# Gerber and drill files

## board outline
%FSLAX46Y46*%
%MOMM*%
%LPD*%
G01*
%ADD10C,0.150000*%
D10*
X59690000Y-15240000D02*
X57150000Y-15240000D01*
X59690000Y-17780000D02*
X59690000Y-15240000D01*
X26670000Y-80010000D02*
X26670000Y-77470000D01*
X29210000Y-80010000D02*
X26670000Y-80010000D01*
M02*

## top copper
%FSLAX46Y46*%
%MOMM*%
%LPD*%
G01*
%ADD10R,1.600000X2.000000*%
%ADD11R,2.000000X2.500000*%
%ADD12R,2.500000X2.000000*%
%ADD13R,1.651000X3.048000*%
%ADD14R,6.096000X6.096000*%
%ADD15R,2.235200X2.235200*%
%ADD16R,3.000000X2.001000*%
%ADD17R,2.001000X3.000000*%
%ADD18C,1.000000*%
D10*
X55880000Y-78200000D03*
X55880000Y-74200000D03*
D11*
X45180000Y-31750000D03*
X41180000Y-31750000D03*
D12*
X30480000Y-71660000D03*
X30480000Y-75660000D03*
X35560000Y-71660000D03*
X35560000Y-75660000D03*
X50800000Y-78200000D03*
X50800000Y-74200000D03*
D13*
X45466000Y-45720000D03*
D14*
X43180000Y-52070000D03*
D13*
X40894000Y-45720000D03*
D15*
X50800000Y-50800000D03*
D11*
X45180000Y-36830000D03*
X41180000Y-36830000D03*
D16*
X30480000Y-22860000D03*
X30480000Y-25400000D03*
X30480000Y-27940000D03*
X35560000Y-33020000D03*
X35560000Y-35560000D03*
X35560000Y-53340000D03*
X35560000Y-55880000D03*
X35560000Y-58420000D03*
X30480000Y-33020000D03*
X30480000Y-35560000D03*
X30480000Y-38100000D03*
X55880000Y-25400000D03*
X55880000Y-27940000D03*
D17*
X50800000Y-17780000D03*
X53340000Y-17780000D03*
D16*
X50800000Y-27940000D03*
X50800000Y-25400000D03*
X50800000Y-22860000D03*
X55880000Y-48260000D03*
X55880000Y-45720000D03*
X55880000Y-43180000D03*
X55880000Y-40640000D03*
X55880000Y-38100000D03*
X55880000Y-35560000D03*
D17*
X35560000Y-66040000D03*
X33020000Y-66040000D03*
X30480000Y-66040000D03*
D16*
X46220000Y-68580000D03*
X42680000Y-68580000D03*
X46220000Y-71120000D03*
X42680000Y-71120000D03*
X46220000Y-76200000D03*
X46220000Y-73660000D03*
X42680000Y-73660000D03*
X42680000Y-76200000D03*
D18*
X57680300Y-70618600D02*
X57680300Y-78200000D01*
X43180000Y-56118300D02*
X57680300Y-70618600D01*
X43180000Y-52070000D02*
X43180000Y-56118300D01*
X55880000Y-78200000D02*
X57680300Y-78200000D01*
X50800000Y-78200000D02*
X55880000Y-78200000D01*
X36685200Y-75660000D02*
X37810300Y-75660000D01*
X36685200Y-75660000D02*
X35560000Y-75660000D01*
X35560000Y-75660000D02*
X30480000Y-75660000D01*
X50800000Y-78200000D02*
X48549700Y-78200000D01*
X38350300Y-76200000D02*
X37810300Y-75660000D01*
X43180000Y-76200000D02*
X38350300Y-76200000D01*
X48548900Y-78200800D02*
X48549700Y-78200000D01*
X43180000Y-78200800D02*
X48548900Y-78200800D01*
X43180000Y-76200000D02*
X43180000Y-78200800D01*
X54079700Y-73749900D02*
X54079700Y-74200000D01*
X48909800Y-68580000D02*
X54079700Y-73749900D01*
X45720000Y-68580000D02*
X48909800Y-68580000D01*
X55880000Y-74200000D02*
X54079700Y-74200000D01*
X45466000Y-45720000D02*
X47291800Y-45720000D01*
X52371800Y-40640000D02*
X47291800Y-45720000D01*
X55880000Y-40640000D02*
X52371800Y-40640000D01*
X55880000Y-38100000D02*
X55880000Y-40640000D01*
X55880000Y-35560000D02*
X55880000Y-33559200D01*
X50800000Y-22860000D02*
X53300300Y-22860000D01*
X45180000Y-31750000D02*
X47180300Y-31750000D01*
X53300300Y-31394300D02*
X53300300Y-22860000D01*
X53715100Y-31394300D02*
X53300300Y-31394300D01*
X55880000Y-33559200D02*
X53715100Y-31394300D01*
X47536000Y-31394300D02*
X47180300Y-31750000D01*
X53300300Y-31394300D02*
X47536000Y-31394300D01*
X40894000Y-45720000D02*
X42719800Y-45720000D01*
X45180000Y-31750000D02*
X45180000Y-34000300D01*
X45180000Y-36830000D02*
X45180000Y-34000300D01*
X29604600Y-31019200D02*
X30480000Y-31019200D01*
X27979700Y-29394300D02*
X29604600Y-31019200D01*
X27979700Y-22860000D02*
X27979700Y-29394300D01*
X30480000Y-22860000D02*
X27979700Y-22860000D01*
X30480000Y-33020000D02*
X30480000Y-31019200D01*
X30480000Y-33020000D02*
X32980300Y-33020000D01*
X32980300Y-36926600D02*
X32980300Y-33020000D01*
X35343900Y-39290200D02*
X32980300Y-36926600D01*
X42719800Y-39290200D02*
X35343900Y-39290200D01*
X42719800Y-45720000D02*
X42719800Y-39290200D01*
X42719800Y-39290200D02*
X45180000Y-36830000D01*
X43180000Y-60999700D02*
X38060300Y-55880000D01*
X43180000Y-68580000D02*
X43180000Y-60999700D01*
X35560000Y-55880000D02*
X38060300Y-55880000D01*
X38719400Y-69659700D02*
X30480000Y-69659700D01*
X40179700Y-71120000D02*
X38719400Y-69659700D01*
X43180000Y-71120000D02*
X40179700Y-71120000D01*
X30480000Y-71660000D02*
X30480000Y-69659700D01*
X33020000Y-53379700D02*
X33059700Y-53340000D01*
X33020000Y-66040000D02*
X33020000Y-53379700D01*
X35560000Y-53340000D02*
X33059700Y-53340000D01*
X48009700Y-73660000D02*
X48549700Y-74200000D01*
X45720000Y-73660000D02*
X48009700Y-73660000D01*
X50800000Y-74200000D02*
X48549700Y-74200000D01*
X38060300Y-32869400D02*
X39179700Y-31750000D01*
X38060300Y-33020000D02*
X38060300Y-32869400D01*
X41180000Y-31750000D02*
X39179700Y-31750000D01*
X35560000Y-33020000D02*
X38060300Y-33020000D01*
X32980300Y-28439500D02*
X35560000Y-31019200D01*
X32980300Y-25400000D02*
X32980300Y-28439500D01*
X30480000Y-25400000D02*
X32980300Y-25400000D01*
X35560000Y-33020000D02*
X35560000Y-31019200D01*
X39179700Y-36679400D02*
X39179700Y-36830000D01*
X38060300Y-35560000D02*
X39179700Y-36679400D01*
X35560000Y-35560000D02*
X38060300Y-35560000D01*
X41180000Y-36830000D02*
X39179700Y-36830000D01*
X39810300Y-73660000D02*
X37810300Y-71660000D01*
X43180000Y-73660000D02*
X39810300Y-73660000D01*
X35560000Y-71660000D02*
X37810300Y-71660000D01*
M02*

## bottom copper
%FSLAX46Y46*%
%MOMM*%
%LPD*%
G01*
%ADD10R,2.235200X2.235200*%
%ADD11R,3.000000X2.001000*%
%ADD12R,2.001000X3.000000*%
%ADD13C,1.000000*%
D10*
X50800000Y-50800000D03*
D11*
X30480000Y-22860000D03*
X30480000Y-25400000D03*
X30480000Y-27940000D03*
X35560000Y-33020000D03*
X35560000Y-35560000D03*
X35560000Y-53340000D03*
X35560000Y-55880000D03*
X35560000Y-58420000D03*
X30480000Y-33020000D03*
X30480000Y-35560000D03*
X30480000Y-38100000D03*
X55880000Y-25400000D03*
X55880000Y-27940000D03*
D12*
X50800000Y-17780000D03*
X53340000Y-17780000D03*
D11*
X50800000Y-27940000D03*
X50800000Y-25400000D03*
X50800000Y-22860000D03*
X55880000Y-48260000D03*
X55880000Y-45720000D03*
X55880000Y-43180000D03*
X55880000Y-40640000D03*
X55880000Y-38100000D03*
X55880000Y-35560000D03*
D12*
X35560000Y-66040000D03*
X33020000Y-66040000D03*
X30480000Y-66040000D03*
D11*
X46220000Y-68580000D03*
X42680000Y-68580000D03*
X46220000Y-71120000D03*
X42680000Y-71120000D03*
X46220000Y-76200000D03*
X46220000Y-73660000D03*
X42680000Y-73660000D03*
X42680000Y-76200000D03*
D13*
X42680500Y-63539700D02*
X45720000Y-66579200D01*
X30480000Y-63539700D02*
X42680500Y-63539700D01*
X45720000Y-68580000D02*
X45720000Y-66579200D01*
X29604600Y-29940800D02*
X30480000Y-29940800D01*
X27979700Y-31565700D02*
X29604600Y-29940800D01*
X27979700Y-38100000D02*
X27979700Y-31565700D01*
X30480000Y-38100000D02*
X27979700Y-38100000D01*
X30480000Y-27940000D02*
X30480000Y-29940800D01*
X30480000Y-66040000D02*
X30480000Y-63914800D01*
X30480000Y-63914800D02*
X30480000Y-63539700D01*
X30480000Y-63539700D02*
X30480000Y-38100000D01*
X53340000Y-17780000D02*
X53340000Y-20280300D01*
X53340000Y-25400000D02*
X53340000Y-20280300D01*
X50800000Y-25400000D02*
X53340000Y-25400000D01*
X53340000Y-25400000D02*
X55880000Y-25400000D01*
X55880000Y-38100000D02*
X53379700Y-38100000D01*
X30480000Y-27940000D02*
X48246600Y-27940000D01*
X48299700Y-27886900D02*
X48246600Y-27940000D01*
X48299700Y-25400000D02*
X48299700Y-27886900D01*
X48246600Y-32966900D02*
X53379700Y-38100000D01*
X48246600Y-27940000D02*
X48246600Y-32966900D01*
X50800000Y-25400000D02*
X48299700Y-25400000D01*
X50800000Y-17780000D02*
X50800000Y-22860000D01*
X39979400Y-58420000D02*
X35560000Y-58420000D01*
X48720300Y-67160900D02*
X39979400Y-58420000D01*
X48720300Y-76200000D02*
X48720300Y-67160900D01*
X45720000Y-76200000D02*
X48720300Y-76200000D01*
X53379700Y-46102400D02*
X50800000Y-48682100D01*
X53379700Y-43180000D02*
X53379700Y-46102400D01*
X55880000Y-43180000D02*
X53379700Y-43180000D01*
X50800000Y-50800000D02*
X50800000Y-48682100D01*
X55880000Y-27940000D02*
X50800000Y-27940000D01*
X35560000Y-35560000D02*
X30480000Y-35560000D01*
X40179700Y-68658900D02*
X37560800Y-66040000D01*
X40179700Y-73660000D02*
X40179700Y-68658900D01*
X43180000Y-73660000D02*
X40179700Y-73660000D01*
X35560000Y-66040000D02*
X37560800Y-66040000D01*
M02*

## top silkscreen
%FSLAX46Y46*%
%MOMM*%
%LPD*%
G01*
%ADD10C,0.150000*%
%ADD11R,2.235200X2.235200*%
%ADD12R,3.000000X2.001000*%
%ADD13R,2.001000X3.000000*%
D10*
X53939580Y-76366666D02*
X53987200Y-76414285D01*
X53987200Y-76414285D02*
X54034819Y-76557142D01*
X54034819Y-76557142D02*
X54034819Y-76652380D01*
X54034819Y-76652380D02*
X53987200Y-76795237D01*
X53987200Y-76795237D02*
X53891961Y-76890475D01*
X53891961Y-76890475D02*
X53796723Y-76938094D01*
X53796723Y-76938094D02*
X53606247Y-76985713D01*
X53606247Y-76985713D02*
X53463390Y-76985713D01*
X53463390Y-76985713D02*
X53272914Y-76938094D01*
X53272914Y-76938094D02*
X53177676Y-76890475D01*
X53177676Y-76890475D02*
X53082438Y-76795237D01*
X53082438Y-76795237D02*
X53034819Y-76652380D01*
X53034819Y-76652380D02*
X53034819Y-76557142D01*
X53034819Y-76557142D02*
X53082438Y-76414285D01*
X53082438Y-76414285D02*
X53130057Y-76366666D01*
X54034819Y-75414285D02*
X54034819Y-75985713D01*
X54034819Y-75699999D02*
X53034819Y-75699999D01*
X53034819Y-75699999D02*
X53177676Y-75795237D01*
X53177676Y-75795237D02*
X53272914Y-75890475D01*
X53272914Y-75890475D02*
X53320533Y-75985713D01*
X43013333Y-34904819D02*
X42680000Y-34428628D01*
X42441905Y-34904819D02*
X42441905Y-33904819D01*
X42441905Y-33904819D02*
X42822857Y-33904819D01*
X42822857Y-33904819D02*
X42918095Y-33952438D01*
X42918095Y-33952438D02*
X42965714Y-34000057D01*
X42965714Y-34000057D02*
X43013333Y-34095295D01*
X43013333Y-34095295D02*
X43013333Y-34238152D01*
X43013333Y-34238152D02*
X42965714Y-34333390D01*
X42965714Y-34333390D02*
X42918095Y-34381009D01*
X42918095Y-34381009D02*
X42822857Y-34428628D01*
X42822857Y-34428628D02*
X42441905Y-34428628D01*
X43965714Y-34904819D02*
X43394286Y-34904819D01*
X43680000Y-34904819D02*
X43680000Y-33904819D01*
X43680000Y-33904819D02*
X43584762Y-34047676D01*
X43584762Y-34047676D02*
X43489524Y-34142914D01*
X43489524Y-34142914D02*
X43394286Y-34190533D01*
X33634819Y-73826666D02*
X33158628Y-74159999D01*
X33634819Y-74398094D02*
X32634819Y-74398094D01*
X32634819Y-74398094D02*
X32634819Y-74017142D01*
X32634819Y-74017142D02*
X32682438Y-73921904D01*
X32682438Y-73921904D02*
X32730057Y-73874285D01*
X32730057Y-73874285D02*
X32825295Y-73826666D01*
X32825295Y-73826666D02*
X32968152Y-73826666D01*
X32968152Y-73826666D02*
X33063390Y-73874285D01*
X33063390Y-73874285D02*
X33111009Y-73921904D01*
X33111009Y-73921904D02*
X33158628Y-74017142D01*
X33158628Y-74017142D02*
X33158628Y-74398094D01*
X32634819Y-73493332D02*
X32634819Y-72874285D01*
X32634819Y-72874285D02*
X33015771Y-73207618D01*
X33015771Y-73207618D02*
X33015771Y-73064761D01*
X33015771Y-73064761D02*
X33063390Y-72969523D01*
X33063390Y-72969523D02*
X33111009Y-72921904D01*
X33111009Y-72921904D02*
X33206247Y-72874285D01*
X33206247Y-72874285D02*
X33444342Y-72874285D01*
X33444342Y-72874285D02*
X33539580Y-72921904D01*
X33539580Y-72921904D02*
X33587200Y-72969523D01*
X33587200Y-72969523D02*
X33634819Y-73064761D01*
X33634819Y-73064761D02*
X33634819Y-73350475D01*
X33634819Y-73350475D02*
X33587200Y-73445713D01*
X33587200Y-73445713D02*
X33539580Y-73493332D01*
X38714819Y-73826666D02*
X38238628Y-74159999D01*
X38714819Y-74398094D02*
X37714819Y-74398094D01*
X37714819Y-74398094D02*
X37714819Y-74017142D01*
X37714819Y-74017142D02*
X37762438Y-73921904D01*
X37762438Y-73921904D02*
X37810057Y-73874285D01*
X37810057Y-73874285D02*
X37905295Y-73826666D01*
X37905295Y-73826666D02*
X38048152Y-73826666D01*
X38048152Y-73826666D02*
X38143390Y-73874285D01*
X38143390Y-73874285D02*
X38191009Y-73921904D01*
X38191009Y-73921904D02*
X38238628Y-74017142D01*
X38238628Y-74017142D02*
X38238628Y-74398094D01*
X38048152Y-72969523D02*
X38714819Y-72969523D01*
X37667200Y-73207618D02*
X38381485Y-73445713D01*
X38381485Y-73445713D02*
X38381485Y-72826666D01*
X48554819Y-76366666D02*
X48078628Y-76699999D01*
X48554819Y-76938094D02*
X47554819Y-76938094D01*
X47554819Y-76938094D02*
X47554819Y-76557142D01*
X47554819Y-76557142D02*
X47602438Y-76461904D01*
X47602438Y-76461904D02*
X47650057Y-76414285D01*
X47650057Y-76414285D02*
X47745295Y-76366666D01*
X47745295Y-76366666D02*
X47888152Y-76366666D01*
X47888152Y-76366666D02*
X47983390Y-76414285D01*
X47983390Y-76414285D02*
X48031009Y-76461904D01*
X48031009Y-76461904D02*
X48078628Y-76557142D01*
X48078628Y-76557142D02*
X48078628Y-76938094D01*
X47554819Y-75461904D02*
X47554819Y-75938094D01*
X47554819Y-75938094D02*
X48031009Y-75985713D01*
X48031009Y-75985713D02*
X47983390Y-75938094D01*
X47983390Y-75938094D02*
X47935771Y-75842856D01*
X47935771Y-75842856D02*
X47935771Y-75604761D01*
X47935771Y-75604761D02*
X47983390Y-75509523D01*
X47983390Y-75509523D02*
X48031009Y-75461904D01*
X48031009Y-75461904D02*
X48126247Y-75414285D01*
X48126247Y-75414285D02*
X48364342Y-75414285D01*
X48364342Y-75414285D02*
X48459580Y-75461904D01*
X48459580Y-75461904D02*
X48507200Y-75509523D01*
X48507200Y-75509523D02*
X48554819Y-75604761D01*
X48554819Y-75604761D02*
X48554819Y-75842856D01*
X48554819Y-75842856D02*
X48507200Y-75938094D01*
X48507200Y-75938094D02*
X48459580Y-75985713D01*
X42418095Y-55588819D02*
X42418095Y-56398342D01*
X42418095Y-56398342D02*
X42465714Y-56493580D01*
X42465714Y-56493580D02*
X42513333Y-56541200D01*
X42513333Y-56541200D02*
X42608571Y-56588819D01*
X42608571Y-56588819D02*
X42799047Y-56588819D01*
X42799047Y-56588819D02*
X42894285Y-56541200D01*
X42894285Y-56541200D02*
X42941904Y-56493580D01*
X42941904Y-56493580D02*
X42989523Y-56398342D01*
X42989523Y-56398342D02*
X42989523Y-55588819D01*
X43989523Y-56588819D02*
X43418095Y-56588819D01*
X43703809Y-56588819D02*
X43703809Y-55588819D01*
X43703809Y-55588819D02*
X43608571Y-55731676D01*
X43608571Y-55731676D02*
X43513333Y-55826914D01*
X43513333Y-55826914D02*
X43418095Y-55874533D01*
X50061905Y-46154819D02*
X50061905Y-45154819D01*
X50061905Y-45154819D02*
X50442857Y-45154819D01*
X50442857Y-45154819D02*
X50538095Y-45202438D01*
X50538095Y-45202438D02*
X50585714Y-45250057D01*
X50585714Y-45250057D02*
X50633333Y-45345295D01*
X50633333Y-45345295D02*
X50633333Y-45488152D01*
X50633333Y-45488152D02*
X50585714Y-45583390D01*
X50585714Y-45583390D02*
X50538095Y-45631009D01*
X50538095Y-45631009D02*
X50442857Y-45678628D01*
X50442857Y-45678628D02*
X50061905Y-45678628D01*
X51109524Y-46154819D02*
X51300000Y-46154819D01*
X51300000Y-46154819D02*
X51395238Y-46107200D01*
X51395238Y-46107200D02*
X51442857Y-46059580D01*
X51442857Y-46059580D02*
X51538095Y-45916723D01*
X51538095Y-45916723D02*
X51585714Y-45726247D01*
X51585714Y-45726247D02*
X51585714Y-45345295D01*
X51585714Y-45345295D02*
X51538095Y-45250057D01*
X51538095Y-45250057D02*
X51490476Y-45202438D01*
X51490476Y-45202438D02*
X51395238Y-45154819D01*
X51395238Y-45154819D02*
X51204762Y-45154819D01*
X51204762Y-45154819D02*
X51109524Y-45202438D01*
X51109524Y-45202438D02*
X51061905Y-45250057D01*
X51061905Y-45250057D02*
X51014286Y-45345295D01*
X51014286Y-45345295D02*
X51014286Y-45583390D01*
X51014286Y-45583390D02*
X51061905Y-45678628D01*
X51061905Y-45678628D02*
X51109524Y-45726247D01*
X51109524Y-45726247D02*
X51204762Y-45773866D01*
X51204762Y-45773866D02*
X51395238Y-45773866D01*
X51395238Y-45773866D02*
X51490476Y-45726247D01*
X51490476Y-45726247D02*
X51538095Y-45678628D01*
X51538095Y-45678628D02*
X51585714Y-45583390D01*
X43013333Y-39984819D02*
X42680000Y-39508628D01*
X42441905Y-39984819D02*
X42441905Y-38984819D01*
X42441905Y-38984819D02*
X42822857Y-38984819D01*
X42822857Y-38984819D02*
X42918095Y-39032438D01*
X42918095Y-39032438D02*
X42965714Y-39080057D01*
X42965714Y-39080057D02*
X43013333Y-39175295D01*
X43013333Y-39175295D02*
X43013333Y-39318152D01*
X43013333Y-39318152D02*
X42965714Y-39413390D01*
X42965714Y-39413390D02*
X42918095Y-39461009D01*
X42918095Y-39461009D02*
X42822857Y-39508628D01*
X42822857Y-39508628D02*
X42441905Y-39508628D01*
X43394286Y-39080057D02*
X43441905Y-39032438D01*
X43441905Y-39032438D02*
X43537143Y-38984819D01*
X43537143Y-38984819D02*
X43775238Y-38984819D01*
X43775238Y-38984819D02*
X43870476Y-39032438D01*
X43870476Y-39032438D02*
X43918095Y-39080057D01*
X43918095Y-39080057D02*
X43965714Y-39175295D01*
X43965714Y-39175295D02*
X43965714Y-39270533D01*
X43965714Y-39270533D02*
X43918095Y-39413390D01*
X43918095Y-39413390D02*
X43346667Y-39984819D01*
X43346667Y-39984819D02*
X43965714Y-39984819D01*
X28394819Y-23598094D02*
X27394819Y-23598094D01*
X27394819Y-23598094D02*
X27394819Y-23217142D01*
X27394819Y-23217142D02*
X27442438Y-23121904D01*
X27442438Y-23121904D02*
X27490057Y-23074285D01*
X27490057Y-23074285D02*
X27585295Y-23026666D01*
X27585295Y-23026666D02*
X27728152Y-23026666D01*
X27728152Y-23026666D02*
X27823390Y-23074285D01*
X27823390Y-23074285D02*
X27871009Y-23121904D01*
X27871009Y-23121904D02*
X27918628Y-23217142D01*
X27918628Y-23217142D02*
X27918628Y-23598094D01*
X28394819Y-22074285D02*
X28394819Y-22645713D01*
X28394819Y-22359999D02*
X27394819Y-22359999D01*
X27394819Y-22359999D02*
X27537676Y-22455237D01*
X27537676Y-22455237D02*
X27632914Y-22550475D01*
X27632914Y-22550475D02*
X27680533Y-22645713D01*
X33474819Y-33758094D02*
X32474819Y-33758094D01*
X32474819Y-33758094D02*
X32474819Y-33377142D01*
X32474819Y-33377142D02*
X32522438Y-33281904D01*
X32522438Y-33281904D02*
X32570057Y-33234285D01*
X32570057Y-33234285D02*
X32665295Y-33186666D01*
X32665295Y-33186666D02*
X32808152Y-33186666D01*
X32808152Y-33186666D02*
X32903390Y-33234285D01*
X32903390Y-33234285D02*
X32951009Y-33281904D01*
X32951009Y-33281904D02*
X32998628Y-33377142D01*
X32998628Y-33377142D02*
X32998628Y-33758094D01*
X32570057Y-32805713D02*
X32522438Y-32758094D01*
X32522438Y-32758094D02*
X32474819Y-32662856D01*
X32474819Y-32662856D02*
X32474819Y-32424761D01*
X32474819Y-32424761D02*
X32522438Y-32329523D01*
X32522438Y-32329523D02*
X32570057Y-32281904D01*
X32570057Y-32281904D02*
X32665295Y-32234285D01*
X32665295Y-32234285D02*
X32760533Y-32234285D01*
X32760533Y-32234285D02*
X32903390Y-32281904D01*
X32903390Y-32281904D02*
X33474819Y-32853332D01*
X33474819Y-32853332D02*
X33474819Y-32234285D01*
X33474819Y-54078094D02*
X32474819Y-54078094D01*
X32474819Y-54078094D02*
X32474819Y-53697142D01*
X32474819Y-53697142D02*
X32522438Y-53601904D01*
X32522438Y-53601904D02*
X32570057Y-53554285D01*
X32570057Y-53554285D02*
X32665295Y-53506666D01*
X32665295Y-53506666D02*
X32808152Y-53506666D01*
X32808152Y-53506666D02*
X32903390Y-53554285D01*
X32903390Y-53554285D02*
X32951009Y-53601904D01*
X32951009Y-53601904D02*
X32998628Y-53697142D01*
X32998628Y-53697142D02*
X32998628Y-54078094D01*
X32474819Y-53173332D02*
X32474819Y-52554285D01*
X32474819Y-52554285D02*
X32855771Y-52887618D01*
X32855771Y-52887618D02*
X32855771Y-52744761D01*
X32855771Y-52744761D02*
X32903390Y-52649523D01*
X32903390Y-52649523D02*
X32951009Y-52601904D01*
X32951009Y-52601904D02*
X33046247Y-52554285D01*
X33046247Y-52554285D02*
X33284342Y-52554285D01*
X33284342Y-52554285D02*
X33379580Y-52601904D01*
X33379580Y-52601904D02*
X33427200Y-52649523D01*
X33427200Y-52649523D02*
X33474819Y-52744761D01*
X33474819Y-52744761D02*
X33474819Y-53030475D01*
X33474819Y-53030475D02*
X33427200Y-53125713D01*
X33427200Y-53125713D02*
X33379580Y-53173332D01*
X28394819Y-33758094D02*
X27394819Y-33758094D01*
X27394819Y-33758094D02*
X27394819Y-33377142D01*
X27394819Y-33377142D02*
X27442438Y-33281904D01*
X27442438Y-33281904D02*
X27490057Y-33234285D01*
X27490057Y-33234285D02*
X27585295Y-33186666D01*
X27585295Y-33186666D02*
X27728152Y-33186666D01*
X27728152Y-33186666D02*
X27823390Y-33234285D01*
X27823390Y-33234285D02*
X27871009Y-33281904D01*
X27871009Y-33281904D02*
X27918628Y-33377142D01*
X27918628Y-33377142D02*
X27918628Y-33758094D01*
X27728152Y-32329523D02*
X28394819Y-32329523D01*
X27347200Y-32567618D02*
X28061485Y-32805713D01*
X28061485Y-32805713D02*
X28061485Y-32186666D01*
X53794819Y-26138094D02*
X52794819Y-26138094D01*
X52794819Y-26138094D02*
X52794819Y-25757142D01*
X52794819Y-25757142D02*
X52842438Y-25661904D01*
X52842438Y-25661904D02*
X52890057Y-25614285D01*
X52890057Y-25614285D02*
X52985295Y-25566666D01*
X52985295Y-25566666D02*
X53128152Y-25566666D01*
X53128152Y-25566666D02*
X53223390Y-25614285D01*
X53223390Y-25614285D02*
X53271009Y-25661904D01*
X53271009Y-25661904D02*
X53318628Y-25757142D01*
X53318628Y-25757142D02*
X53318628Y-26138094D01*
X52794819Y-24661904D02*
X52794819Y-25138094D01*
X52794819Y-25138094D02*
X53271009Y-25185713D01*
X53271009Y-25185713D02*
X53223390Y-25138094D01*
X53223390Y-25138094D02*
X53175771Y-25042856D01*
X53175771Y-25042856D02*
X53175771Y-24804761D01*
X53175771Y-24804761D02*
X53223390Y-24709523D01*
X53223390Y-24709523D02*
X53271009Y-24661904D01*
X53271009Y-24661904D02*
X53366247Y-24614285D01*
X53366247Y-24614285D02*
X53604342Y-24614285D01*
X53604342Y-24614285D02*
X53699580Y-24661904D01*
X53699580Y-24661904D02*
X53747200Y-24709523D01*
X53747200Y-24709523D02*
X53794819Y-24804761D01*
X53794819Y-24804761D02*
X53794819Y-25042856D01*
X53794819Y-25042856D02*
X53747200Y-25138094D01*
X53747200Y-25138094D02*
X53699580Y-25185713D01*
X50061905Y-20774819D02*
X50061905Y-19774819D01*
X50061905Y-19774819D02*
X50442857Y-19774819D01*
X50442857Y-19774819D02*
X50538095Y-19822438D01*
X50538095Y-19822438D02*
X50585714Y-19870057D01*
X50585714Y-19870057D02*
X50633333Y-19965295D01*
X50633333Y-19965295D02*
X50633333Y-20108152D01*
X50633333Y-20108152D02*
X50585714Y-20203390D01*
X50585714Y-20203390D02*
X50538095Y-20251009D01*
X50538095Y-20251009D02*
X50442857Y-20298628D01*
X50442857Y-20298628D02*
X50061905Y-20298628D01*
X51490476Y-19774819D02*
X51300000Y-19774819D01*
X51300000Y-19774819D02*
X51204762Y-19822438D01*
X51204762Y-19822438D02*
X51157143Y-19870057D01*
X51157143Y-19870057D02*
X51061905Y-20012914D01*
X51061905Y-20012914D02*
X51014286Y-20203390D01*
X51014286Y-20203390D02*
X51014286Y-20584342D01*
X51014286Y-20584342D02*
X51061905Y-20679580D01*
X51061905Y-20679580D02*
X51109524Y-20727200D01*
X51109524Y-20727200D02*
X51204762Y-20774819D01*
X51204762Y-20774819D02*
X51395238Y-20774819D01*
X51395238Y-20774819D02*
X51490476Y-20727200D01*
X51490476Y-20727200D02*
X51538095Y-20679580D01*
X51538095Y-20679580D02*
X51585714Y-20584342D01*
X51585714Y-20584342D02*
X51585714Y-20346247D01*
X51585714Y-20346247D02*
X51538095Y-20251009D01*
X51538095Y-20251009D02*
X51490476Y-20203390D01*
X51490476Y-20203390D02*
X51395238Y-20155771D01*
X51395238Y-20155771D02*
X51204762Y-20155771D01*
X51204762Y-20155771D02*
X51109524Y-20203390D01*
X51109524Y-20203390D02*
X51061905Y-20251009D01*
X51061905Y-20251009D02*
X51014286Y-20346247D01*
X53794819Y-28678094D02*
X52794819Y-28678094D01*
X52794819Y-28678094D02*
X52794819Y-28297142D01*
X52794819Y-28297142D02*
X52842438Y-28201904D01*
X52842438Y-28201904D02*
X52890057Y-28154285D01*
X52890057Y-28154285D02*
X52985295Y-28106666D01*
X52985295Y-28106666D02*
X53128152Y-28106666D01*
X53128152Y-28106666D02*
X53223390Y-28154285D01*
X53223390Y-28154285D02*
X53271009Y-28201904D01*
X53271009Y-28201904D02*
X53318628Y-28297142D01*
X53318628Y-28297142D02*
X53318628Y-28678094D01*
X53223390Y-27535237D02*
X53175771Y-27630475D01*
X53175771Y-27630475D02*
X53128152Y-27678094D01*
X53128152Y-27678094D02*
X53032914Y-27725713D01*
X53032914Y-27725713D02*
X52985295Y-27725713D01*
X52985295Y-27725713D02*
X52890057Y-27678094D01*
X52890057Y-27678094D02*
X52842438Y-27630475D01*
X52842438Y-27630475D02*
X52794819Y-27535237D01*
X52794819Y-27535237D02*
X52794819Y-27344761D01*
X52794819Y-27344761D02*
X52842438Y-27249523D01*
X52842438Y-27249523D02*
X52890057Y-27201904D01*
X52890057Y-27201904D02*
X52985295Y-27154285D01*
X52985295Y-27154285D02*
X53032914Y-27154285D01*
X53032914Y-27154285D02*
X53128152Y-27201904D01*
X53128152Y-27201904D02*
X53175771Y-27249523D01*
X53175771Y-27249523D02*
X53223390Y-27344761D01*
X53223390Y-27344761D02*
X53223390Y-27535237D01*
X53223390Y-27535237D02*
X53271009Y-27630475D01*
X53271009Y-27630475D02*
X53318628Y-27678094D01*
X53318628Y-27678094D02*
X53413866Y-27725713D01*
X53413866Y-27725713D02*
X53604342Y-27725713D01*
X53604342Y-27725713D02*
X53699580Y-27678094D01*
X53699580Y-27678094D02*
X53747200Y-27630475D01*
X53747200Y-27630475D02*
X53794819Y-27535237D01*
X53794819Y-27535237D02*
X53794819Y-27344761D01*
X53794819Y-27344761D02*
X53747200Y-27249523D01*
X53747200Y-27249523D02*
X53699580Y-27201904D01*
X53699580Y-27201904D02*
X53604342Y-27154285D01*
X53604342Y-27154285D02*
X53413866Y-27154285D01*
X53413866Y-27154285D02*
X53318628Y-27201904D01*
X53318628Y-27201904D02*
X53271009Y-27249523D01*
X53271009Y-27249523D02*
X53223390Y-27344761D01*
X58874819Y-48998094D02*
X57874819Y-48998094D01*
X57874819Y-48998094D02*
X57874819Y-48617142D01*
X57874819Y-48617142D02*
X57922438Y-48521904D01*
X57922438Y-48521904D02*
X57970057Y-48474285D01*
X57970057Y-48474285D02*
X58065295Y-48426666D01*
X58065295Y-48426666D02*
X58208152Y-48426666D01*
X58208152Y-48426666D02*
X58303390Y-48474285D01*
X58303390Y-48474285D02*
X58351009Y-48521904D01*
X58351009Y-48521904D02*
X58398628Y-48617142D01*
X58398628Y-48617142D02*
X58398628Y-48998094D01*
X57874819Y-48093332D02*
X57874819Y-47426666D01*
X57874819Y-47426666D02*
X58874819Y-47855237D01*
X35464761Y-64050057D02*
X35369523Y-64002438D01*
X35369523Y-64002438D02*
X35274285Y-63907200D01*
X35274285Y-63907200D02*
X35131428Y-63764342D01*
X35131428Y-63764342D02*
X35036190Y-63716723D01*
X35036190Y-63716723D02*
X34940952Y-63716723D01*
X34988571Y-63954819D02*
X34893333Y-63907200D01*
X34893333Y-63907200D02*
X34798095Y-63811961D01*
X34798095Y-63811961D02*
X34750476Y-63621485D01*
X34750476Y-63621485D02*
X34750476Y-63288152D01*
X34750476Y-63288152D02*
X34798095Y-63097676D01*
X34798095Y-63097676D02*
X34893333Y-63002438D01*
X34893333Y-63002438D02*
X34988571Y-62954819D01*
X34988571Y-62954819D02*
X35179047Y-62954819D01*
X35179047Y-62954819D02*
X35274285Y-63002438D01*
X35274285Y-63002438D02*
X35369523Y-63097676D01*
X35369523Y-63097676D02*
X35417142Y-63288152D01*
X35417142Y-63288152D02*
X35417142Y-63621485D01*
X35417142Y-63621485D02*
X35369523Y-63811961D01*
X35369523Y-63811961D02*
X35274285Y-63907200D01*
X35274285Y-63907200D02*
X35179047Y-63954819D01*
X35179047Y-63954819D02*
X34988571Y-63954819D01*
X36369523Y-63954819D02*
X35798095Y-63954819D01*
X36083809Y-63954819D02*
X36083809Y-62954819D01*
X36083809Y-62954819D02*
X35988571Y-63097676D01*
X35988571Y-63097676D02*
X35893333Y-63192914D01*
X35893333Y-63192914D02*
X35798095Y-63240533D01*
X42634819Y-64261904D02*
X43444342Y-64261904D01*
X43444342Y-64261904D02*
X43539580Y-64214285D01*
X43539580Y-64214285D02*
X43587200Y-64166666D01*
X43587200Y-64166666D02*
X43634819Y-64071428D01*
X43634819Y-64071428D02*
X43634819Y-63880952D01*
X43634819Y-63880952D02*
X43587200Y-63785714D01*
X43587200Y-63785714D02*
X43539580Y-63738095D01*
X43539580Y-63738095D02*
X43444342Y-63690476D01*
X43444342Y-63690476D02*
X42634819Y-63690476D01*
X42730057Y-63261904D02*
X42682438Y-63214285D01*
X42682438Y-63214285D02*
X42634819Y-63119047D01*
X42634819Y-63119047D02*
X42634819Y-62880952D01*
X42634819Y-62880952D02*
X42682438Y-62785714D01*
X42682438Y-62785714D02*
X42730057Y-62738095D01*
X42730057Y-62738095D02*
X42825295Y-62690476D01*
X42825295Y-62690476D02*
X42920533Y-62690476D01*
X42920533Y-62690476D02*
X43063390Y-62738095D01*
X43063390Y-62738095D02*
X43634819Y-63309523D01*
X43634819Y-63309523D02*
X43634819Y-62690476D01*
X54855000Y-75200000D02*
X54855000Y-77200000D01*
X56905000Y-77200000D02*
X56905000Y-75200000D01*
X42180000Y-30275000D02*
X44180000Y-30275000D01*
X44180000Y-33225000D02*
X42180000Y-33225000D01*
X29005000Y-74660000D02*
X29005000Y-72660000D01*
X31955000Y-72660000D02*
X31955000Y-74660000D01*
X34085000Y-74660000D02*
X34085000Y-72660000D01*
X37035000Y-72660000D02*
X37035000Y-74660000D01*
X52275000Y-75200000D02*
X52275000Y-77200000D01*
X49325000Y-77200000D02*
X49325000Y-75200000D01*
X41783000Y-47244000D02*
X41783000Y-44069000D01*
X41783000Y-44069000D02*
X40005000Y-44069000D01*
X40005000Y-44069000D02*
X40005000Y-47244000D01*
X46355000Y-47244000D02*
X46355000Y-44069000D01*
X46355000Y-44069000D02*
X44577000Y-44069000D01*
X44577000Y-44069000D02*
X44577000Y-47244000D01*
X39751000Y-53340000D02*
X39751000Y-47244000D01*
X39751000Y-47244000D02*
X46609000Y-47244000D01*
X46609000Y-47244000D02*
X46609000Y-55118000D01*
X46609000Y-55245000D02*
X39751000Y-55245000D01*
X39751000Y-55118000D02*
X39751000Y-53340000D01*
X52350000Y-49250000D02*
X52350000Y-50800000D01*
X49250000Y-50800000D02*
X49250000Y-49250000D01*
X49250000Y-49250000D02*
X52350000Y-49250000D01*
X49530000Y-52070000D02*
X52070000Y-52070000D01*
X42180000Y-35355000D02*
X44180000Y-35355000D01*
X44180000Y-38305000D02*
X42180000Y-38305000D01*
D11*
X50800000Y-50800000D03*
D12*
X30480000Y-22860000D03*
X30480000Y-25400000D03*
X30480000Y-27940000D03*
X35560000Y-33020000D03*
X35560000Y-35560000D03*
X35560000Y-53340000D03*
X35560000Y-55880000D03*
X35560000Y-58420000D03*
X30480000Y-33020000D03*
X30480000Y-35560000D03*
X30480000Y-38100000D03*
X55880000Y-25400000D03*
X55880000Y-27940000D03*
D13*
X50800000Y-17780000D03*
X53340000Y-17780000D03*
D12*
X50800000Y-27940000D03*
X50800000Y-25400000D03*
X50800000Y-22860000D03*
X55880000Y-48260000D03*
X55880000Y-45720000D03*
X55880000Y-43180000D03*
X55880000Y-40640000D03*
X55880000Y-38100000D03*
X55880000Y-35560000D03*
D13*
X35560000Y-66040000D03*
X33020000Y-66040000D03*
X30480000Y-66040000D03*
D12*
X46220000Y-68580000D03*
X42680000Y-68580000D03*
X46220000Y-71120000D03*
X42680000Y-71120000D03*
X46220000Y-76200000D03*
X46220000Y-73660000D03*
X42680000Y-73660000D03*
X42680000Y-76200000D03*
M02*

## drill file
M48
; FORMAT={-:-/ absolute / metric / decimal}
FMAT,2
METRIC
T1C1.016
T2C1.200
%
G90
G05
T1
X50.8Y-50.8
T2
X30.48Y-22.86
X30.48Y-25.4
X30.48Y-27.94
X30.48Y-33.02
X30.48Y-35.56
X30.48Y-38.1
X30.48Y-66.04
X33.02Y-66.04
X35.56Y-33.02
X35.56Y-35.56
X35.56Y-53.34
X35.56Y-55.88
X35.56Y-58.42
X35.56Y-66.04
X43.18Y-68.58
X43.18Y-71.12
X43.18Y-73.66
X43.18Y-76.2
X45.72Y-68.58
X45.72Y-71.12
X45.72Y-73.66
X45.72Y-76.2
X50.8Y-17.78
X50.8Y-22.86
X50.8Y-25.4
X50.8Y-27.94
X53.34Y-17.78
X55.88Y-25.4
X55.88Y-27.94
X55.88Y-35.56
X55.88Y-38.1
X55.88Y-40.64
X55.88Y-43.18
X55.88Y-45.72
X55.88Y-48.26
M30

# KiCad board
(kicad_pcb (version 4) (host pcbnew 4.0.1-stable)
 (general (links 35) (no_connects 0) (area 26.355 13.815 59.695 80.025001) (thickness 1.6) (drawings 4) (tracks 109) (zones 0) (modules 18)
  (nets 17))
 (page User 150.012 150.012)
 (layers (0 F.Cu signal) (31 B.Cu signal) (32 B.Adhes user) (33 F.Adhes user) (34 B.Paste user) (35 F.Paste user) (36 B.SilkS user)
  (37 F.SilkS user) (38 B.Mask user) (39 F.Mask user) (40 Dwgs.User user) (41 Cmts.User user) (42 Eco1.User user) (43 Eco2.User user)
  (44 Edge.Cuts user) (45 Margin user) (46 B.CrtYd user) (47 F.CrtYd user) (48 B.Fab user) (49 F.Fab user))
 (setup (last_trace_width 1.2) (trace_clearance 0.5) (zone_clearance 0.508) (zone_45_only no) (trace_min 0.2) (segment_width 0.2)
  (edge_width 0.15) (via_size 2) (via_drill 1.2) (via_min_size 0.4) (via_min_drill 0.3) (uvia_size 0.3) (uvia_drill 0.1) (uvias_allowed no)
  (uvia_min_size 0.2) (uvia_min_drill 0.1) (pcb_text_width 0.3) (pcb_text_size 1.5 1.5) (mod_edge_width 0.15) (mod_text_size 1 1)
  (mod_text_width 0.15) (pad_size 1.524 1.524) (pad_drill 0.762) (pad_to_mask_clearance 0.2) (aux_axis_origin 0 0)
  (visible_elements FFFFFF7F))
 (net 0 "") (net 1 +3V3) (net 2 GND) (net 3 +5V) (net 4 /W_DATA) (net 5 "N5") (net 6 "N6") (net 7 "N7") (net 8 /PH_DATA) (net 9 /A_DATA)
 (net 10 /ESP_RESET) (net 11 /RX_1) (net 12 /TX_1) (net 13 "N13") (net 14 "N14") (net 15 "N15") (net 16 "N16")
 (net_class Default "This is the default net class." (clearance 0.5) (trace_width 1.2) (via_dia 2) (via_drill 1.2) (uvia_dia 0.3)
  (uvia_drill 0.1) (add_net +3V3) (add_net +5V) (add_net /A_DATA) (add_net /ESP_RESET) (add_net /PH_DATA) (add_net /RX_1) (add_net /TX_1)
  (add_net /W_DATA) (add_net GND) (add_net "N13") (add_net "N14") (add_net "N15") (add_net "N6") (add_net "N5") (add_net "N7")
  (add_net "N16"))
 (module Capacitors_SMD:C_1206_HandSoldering (layer F.Cu) (at 55.88 76.2 90)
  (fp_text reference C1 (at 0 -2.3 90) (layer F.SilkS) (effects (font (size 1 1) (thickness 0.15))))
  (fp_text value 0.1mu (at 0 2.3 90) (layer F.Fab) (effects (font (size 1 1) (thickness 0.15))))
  (fp_line (start 1 -1.025) (end -1 -1.025) (layer F.SilkS) (width 0.15))
  (fp_line (start -1 1.025) (end 1 1.025) (layer F.SilkS) (width 0.15))
  (pad 1 smd rect (at -2 0 90) (size 2 1.6) (layers F.Cu F.Paste F.Mask) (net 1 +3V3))
  (pad 2 smd rect (at 2 0 90) (size 2 1.6) (layers F.Cu F.Paste F.Mask) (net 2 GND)))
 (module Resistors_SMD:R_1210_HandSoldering (layer F.Cu) (at 43.18 31.75 180)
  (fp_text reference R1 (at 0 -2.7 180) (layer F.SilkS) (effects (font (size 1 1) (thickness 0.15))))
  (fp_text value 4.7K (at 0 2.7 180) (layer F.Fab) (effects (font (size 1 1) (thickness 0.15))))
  (fp_line (start 1 1.475) (end -1 1.475) (layer F.SilkS) (width 0.15))
  (fp_line (start -1 -1.475) (end 1 -1.475) (layer F.SilkS) (width 0.15))
  (pad 1 smd rect (at -2 0 180) (size 2 2.5) (layers F.Cu F.Paste F.Mask) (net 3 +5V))
  (pad 2 smd rect (at 2 0 180) (size 2 2.5) (layers F.Cu F.Paste F.Mask) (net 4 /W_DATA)))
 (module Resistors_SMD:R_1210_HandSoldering (layer F.Cu) (at 30.48 73.66 270)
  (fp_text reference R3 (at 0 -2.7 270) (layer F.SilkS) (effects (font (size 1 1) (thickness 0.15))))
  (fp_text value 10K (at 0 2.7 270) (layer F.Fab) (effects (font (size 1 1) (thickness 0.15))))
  (fp_line (start 1 1.475) (end -1 1.475) (layer F.SilkS) (width 0.15))
  (fp_line (start -1 -1.475) (end 1 -1.475) (layer F.SilkS) (width 0.15))
  (pad 1 smd rect (at -2 0 270) (size 2 2.5) (layers F.Cu F.Paste F.Mask) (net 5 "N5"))
  (pad 2 smd rect (at 2 0 270) (size 2 2.5) (layers F.Cu F.Paste F.Mask) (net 1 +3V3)))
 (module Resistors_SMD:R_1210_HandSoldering (layer F.Cu) (at 35.56 73.66 270)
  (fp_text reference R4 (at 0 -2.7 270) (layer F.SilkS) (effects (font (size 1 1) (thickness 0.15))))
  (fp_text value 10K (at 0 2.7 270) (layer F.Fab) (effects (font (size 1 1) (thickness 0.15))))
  (fp_line (start 1 1.475) (end -1 1.475) (layer F.SilkS) (width 0.15))
  (fp_line (start -1 -1.475) (end 1 -1.475) (layer F.SilkS) (width 0.15))
  (pad 1 smd rect (at -2 0 270) (size 2 2.5) (layers F.Cu F.Paste F.Mask) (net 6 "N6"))
  (pad 2 smd rect (at 2 0 270) (size 2 2.5) (layers F.Cu F.Paste F.Mask) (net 1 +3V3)))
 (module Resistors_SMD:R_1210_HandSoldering (layer F.Cu) (at 50.8 76.2 90)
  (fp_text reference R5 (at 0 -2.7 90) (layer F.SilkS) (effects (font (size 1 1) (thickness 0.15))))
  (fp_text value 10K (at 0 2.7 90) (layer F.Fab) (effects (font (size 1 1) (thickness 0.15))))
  (fp_line (start 1 1.475) (end -1 1.475) (layer F.SilkS) (width 0.15))
  (fp_line (start -1 -1.475) (end 1 -1.475) (layer F.SilkS) (width 0.15))
  (pad 1 smd rect (at -2 0 90) (size 2 2.5) (layers F.Cu F.Paste F.Mask) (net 1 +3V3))
  (pad 2 smd rect (at 2 0 90) (size 2 2.5) (layers F.Cu F.Paste F.Mask) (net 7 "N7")))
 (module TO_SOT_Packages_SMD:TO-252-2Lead (layer F.Cu) (at 43.18 45.72 180)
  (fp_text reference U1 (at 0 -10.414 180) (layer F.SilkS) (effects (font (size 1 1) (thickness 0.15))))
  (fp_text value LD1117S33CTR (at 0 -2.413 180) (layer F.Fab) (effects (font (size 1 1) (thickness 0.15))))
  (fp_line (start 1.397 -1.524) (end 1.397 1.651) (layer F.SilkS) (width 0.15))
  (fp_line (start 1.397 1.651) (end 3.175 1.651) (layer F.SilkS) (width 0.15))
  (fp_line (start 3.175 1.651) (end 3.175 -1.524) (layer F.SilkS) (width 0.15))
  (fp_line (start -3.175 -1.524) (end -3.175 1.651) (layer F.SilkS) (width 0.15))
  (fp_line (start -3.175 1.651) (end -1.397 1.651) (layer F.SilkS) (width 0.15))
  (fp_line (start -1.397 1.651) (end -1.397 -1.524) (layer F.SilkS) (width 0.15))
  (fp_line (start 3.429 -7.62) (end 3.429 -1.524) (layer F.SilkS) (width 0.15))
  (fp_line (start 3.429 -1.524) (end -3.429 -1.524) (layer F.SilkS) (width 0.15))
  (fp_line (start -3.429 -1.524) (end -3.429 -9.398) (layer F.SilkS) (width 0.15))
  (fp_line (start -3.429 -9.525) (end 3.429 -9.525) (layer F.SilkS) (width 0.15))
  (fp_line (start 3.429 -9.398) (end 3.429 -7.62) (layer F.SilkS) (width 0.15))
  (pad 1 smd rect (at -2.286 0 180) (size 1.651 3.048) (layers F.Cu F.Paste F.Mask) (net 2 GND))
  (pad 2 smd rect (at 0 -6.35 180) (size 6.096 6.096) (layers F.Cu F.Paste F.Mask) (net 1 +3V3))
  (pad 3 smd rect (at 2.286 0 180) (size 1.651 3.048) (layers F.Cu F.Paste F.Mask) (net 3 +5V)))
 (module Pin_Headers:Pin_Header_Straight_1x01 (layer F.Cu) (at 50.8 50.8)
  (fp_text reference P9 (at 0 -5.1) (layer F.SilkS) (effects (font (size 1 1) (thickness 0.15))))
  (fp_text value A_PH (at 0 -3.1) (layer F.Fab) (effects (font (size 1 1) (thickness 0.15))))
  (fp_line (start 1.55 -1.55) (end 1.55 0) (layer F.SilkS) (width 0.15))
  (fp_line (start -1.55 0) (end -1.55 -1.55) (layer F.SilkS) (width 0.15))
  (fp_line (start -1.55 -1.55) (end 1.55 -1.55) (layer F.SilkS) (width 0.15))
  (fp_line (start -1.27 1.27) (end 1.27 1.27) (layer F.SilkS) (width 0.15))
  (pad 1 thru_hole rect (at 0 0) (size 2.2352 2.2352) (drill 1.016) (layers *.Cu *.Mask F.SilkS) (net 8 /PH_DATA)))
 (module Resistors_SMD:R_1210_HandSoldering (layer F.Cu) (at 43.18 36.83 180)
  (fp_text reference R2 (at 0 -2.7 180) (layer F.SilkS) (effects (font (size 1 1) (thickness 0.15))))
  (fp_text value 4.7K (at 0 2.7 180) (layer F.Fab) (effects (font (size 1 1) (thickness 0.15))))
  (fp_line (start 1 1.475) (end -1 1.475) (layer F.SilkS) (width 0.15))
  (fp_line (start -1 -1.475) (end 1 -1.475) (layer F.SilkS) (width 0.15))
  (pad 1 smd rect (at -2 0 180) (size 2 2.5) (layers F.Cu F.Paste F.Mask) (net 3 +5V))
  (pad 2 smd rect (at 2 0 180) (size 2 2.5) (layers F.Cu F.Paste F.Mask) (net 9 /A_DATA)))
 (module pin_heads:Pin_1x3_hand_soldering (layer F.Cu) (at 30.48 22.86 270)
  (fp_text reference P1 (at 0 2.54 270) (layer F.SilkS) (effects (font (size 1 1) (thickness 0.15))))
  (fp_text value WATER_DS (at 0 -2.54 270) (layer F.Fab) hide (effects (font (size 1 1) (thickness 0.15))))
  (pad 1 thru_hole rect (at 0 0 270) (size 2.001 3) (drill 1.2) (layers *.Cu *.Mask F.SilkS) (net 3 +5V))
  (pad 2 thru_hole rect (at 2.54 0 270) (size 2.001 3) (drill 1.2) (layers *.Cu *.Mask F.SilkS) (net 4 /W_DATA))
  (pad 3 thru_hole rect (at 5.08 0 270) (size 2.001 3) (drill 1.2) (layers *.Cu *.Mask F.SilkS) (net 2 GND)))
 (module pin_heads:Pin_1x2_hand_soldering (layer F.Cu) (at 35.56 33.02 270)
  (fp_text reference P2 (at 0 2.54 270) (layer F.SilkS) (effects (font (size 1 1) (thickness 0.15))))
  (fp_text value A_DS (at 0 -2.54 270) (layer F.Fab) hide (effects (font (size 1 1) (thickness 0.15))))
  (pad 1 thru_hole rect (at 0 0 270) (size 2.001 3) (drill 1.2) (layers *.Cu *.Mask F.SilkS) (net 4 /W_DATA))
  (pad 2 thru_hole rect (at 2.54 0 270) (size 2.001 3) (drill 1.2) (layers *.Cu *.Mask F.SilkS) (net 9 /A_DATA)))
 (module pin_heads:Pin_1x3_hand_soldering (layer F.Cu) (at 35.56 53.34 270)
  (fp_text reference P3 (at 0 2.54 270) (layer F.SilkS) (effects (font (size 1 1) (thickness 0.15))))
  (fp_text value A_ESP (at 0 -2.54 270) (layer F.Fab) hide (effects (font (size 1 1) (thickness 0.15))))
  (pad 1 thru_hole rect (at 0 0 270) (size 2.001 3) (drill 1.2) (layers *.Cu *.Mask F.SilkS) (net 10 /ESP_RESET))
  (pad 2 thru_hole rect (at 2.54 0 270) (size 2.001 3) (drill 1.2) (layers *.Cu *.Mask F.SilkS) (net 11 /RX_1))
  (pad 3 thru_hole rect (at 5.08 0 270) (size 2.001 3) (drill 1.2) (layers *.Cu *.Mask F.SilkS) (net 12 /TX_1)))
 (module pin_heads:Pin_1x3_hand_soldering (layer F.Cu) (at 30.48 33.02 270)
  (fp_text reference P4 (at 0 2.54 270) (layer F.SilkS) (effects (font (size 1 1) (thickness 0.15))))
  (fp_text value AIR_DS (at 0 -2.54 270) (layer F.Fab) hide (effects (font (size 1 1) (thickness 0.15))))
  (pad 1 thru_hole rect (at 0 0 270) (size 2.001 3) (drill 1.2) (layers *.Cu *.Mask F.SilkS) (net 3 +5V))
  (pad 2 thru_hole rect (at 2.54 0 270) (size 2.001 3) (drill 1.2) (layers *.Cu *.Mask F.SilkS) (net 9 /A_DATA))
  (pad 3 thru_hole rect (at 5.08 0 270) (size 2.001 3) (drill 1.2) (layers *.Cu *.Mask F.SilkS) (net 2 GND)))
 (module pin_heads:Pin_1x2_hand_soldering (layer F.Cu) (at 55.88 25.4 270)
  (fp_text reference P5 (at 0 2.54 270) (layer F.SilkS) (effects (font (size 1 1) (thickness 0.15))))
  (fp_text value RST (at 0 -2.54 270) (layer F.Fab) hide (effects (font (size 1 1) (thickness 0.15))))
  (pad 1 thru_hole rect (at 0 0 270) (size 2.001 3) (drill 1.2) (layers *.Cu *.Mask F.SilkS) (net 2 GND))
  (pad 2 thru_hole rect (at 2.54 0 270) (size 2.001 3) (drill 1.2) (layers *.Cu *.Mask F.SilkS) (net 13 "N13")))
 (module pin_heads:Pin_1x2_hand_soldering (layer F.Cu) (at 50.8 17.78)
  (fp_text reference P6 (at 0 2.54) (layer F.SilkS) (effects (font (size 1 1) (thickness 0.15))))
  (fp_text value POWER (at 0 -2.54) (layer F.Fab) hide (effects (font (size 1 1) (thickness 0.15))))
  (pad 1 thru_hole rect (at 0 0) (size 2.001 3) (drill 1.2) (layers *.Cu *.Mask F.SilkS) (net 3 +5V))
  (pad 2 thru_hole rect (at 2.54 0) (size 2.001 3) (drill 1.2) (layers *.Cu *.Mask F.SilkS) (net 2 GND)))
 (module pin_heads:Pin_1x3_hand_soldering (layer F.Cu) (at 50.8 27.94 90)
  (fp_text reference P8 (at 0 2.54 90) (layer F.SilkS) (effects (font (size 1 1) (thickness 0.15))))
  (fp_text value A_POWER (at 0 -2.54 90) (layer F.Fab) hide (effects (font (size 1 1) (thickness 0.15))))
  (pad 1 thru_hole rect (at 0 0 90) (size 2.001 3) (drill 1.2) (layers *.Cu *.Mask F.SilkS) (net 13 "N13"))
  (pad 2 thru_hole rect (at 2.54 0 90) (size 2.001 3) (drill 1.2) (layers *.Cu *.Mask F.SilkS) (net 2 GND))
  (pad 3 thru_hole rect (at 5.08 0 90) (size 2.001 3) (drill 1.2) (layers *.Cu *.Mask F.SilkS) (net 3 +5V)))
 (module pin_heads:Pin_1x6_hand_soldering (layer F.Cu) (at 55.88 48.26 90)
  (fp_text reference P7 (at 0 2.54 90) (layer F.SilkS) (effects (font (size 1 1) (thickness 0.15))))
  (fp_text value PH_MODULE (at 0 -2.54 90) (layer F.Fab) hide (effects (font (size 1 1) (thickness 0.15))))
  (pad 1 thru_hole rect (at 0 0 90) (size 2.001 3) (drill 1.2) (layers *.Cu *.Mask F.SilkS) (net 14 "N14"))
  (pad 2 thru_hole rect (at 2.54 0 90) (size 2.001 3) (drill 1.2) (layers *.Cu *.Mask F.SilkS) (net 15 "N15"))
  (pad 3 thru_hole rect (at 5.08 0 90) (size 2.001 3) (drill 1.2) (layers *.Cu *.Mask F.SilkS) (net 8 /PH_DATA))
  (pad 4 thru_hole rect (at 7.62 0 90) (size 2.001 3) (drill 1.2) (layers *.Cu *.Mask F.SilkS) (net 2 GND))
  (pad 5 thru_hole rect (at 10.16 0 90) (size 2.001 3) (drill 1.2) (layers *.Cu *.Mask F.SilkS) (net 2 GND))
  (pad 6 thru_hole rect (at 12.7 0 90) (size 2.001 3) (drill 1.2) (layers *.Cu *.Mask F.SilkS) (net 3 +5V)))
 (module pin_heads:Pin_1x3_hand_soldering (layer F.Cu) (at 35.56 66.04 180)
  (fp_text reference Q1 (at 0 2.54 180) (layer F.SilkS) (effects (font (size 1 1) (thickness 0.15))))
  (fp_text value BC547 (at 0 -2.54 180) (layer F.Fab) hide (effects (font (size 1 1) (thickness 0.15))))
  (pad 1 thru_hole rect (at 0 0 180) (size 2.001 3) (drill 1.2) (layers *.Cu *.Mask F.SilkS) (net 6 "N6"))
  (pad 2 thru_hole rect (at 2.54 0 180) (size 2.001 3) (drill 1.2) (layers *.Cu *.Mask F.SilkS) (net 10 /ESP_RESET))
  (pad 3 thru_hole rect (at 5.08 0 180) (size 2.001 3) (drill 1.2) (layers *.Cu *.Mask F.SilkS) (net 2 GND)))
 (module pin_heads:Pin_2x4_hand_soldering (layer F.Cu) (at 45.72 68.58 270)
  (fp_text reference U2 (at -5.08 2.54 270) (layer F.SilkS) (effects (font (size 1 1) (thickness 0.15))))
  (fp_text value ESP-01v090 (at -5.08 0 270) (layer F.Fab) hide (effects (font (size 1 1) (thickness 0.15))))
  (pad 2 thru_hole rect (at 0 0 270) (size 2.001 3) (drill 1.2 (offset 0 -0.5)) (layers *.Cu *.Mask F.SilkS) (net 2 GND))
  (pad 1 thru_hole rect (at 0 2.54 270) (size 2.001 3) (drill 1.2 (offset 0 0.5)) (layers *.Cu *.Mask F.SilkS) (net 11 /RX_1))
  (pad 4 thru_hole rect (at 2.54 0 270) (size 2.001 3) (drill 1.2 (offset 0 -0.5)) (layers *.Cu *.Mask F.SilkS) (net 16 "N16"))
  (pad 3 thru_hole rect (at 2.54 2.54 270) (size 2.001 3) (drill 1.2 (offset 0 0.5)) (layers *.Cu *.Mask F.SilkS) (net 5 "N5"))
  (pad 8 thru_hole rect (at 7.62 0 270) (size 2.001 3) (drill 1.2 (offset 0 -0.5)) (layers *.Cu *.Mask F.SilkS) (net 12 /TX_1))
  (pad 6 thru_hole rect (at 5.08 0 270) (size 2.001 3) (drill 1.2 (offset 0 -0.5)) (layers *.Cu *.Mask F.SilkS) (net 7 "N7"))
  (pad 5 thru_hole rect (at 5.08 2.54 270) (size 2.001 3) (drill 1.2 (offset 0 0.5)) (layers *.Cu *.Mask F.SilkS) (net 6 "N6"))
  (pad 7 thru_hole rect (at 7.62 2.54 270) (size 2.001 3) (drill 1.2 (offset 0 0.5)) (layers *.Cu *.Mask F.SilkS) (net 1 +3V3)))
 (gr_line (start 59.69 15.24) (end 57.15 15.24) (layer Edge.Cuts) (width 0.15))
 (gr_line (start 59.69 17.78) (end 59.69 15.24) (layer Edge.Cuts) (width 0.15))
 (gr_line (start 26.67 80.01) (end 26.67 77.47) (layer Edge.Cuts) (width 0.15))
 (gr_line (start 29.21 80.01) (end 26.67 80.01) (layer Edge.Cuts) (width 0.15))
 (segment (start 57.6803 70.6186) (end 57.6803 78.2) (width 1) (layer F.Cu) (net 1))
 (segment (start 43.18 56.1183) (end 57.6803 70.6186) (width 1) (layer F.Cu) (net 1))
 (segment (start 43.18 52.07) (end 43.18 56.1183) (width 1) (layer F.Cu) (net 1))
 (segment (start 55.88 78.2) (end 57.6803 78.2) (width 1) (layer F.Cu) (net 1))
 (segment (start 50.8 78.2) (end 55.88 78.2) (width 1) (layer F.Cu) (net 1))
 (segment (start 36.6852 75.66) (end 37.8103 75.66) (width 1) (layer F.Cu) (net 1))
 (segment (start 36.6852 75.66) (end 35.56 75.66) (width 1) (layer F.Cu) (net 1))
 (segment (start 35.56 75.66) (end 30.48 75.66) (width 1) (layer F.Cu) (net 1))
 (segment (start 50.8 78.2) (end 48.5497 78.2) (width 1) (layer F.Cu) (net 1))
 (segment (start 38.3503 76.2) (end 37.8103 75.66) (width 1) (layer F.Cu) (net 1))
 (segment (start 43.18 76.2) (end 38.3503 76.2) (width 1) (layer F.Cu) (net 1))
 (segment (start 48.5489 78.2008) (end 48.5497 78.2) (width 1) (layer F.Cu) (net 1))
 (segment (start 43.18 78.2008) (end 48.5489 78.2008) (width 1) (layer F.Cu) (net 1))
 (segment (start 43.18 76.2) (end 43.18 78.2008) (width 1) (layer F.Cu) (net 1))
 (segment (start 54.0797 73.7499) (end 54.0797 74.2) (width 1) (layer F.Cu) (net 2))
 (segment (start 48.9098 68.58) (end 54.0797 73.7499) (width 1) (layer F.Cu) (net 2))
 (segment (start 45.72 68.58) (end 48.9098 68.58) (width 1) (layer F.Cu) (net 2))
 (segment (start 55.88 74.2) (end 54.0797 74.2) (width 1) (layer F.Cu) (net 2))
 (segment (start 42.6805 63.5397) (end 45.72 66.5792) (width 1) (layer B.Cu) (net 2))
 (segment (start 30.48 63.5397) (end 42.6805 63.5397) (width 1) (layer B.Cu) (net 2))
 (segment (start 45.72 68.58) (end 45.72 66.5792) (width 1) (layer B.Cu) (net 2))
 (segment (start 29.6046 29.9408) (end 30.48 29.9408) (width 1) (layer B.Cu) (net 2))
 (segment (start 27.9797 31.5657) (end 29.6046 29.9408) (width 1) (layer B.Cu) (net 2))
 (segment (start 27.9797 38.1) (end 27.9797 31.5657) (width 1) (layer B.Cu) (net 2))
 (segment (start 30.48 38.1) (end 27.9797 38.1) (width 1) (layer B.Cu) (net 2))
 (segment (start 30.48 27.94) (end 30.48 29.9408) (width 1) (layer B.Cu) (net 2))
 (segment (start 45.466 45.72) (end 47.2918 45.72) (width 1) (layer F.Cu) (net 2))
 (segment (start 52.3718 40.64) (end 47.2918 45.72) (width 1) (layer F.Cu) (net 2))
 (segment (start 55.88 40.64) (end 52.3718 40.64) (width 1) (layer F.Cu) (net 2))
 (segment (start 30.48 66.04) (end 30.48 63.9148) (width 1) (layer B.Cu) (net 2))
 (segment (start 30.48 63.9148) (end 30.48 63.5397) (width 1) (layer B.Cu) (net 2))
 (segment (start 30.48 63.5397) (end 30.48 38.1) (width 1) (layer B.Cu) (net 2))
 (segment (start 53.34 17.78) (end 53.34 20.2803) (width 1) (layer B.Cu) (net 2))
 (segment (start 53.34 25.4) (end 53.34 20.2803) (width 1) (layer B.Cu) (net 2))
 (segment (start 50.8 25.4) (end 53.34 25.4) (width 1) (layer B.Cu) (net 2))
 (segment (start 53.34 25.4) (end 55.88 25.4) (width 1) (layer B.Cu) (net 2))
 (segment (start 55.88 38.1) (end 53.3797 38.1) (width 1) (layer B.Cu) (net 2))
 (segment (start 30.48 27.94) (end 48.2466 27.94) (width 1) (layer B.Cu) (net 2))
 (segment (start 48.2997 27.8869) (end 48.2466 27.94) (width 1) (layer B.Cu) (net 2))
 (segment (start 48.2997 25.4) (end 48.2997 27.8869) (width 1) (layer B.Cu) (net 2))
 (segment (start 48.2466 32.9669) (end 53.3797 38.1) (width 1) (layer B.Cu) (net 2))
 (segment (start 48.2466 27.94) (end 48.2466 32.9669) (width 1) (layer B.Cu) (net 2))
 (segment (start 50.8 25.4) (end 48.2997 25.4) (width 1) (layer B.Cu) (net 2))
 (segment (start 55.88 38.1) (end 55.88 40.64) (width 1) (layer F.Cu) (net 2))
 (segment (start 55.88 35.56) (end 55.88 33.5592) (width 1) (layer F.Cu) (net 3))
 (segment (start 50.8 22.86) (end 53.3003 22.86) (width 1) (layer F.Cu) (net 3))
 (segment (start 50.8 17.78) (end 50.8 22.86) (width 1) (layer B.Cu) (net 3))
 (segment (start 45.18 31.75) (end 47.1803 31.75) (width 1) (layer F.Cu) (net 3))
 (segment (start 53.3003 31.3943) (end 53.3003 22.86) (width 1) (layer F.Cu) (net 3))
 (segment (start 53.7151 31.3943) (end 53.3003 31.3943) (width 1) (layer F.Cu) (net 3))
 (segment (start 55.88 33.5592) (end 53.7151 31.3943) (width 1) (layer F.Cu) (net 3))
 (segment (start 47.536 31.3943) (end 47.1803 31.75) (width 1) (layer F.Cu) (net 3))
 (segment (start 53.3003 31.3943) (end 47.536 31.3943) (width 1) (layer F.Cu) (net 3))
 (segment (start 40.894 45.72) (end 42.7198 45.72) (width 1) (layer F.Cu) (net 3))
 (segment (start 45.18 31.75) (end 45.18 34.0003) (width 1) (layer F.Cu) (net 3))
 (segment (start 45.18 36.83) (end 45.18 34.0003) (width 1) (layer F.Cu) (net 3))
 (segment (start 29.6046 31.0192) (end 30.48 31.0192) (width 1) (layer F.Cu) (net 3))
 (segment (start 27.9797 29.3943) (end 29.6046 31.0192) (width 1) (layer F.Cu) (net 3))
 (segment (start 27.9797 22.86) (end 27.9797 29.3943) (width 1) (layer F.Cu) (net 3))
 (segment (start 30.48 22.86) (end 27.9797 22.86) (width 1) (layer F.Cu) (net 3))
 (segment (start 30.48 33.02) (end 30.48 31.0192) (width 1) (layer F.Cu) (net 3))
 (segment (start 30.48 33.02) (end 32.9803 33.02) (width 1) (layer F.Cu) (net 3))
 (segment (start 32.9803 36.9266) (end 32.9803 33.02) (width 1) (layer F.Cu) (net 3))
 (segment (start 35.3439 39.2902) (end 32.9803 36.9266) (width 1) (layer F.Cu) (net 3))
 (segment (start 42.7198 39.2902) (end 35.3439 39.2902) (width 1) (layer F.Cu) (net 3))
 (segment (start 42.7198 45.72) (end 42.7198 39.2902) (width 1) (layer F.Cu) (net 3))
 (segment (start 42.7198 39.2902) (end 45.18 36.83) (width 1) (layer F.Cu) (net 3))
 (segment (start 39.9794 58.42) (end 35.56 58.42) (width 1) (layer B.Cu) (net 12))
 (segment (start 48.7203 67.1609) (end 39.9794 58.42) (width 1) (layer B.Cu) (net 12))
 (segment (start 48.7203 76.2) (end 48.7203 67.1609) (width 1) (layer B.Cu) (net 12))
 (segment (start 45.72 76.2) (end 48.7203 76.2) (width 1) (layer B.Cu) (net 12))
 (segment (start 43.18 60.9997) (end 38.0603 55.88) (width 1) (layer F.Cu) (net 11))
 (segment (start 43.18 68.58) (end 43.18 60.9997) (width 1) (layer F.Cu) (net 11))
 (segment (start 35.56 55.88) (end 38.0603 55.88) (width 1) (layer F.Cu) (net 11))
 (segment (start 53.3797 46.1024) (end 50.8 48.6821) (width 1) (layer B.Cu) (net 8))
 (segment (start 53.3797 43.18) (end 53.3797 46.1024) (width 1) (layer B.Cu) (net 8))
 (segment (start 55.88 43.18) (end 53.3797 43.18) (width 1) (layer B.Cu) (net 8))
 (segment (start 50.8 50.8) (end 50.8 48.6821) (width 1) (layer B.Cu) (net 8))
 (segment (start 38.7194 69.6597) (end 30.48 69.6597) (width 1) (layer F.Cu) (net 5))
 (segment (start 40.1797 71.12) (end 38.7194 69.6597) (width 1) (layer F.Cu) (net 5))
 (segment (start 43.18 71.12) (end 40.1797 71.12) (width 1) (layer F.Cu) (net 5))
 (segment (start 30.48 71.66) (end 30.48 69.6597) (width 1) (layer F.Cu) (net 5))
 (segment (start 33.02 53.3797) (end 33.0597 53.34) (width 1) (layer F.Cu) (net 10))
 (segment (start 33.02 66.04) (end 33.02 53.3797) (width 1) (layer F.Cu) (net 10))
 (segment (start 35.56 53.34) (end 33.0597 53.34) (width 1) (layer F.Cu) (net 10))
 (segment (start 48.0097 73.66) (end 48.5497 74.2) (width 1) (layer F.Cu) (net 7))
 (segment (start 45.72 73.66) (end 48.0097 73.66) (width 1) (layer F.Cu) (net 7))
 (segment (start 50.8 74.2) (end 48.5497 74.2) (width 1) (layer F.Cu) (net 7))
 (segment (start 55.88 27.94) (end 50.8 27.94) (width 1) (layer B.Cu) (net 13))
 (segment (start 38.0603 32.8694) (end 39.1797 31.75) (width 1) (layer F.Cu) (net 4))
 (segment (start 38.0603 33.02) (end 38.0603 32.8694) (width 1) (layer F.Cu) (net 4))
 (segment (start 41.18 31.75) (end 39.1797 31.75) (width 1) (layer F.Cu) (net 4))
 (segment (start 35.56 33.02) (end 38.0603 33.02) (width 1) (layer F.Cu) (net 4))
 (segment (start 32.9803 28.4395) (end 35.56 31.0192) (width 1) (layer F.Cu) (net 4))
 (segment (start 32.9803 25.4) (end 32.9803 28.4395) (width 1) (layer F.Cu) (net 4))
 (segment (start 30.48 25.4) (end 32.9803 25.4) (width 1) (layer F.Cu) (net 4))
 (segment (start 35.56 33.02) (end 35.56 31.0192) (width 1) (layer F.Cu) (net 4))
 (segment (start 35.56 35.56) (end 30.48 35.56) (width 1) (layer B.Cu) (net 9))
 (segment (start 39.1797 36.6794) (end 39.1797 36.83) (width 1) (layer F.Cu) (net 9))
 (segment (start 38.0603 35.56) (end 39.1797 36.6794) (width 1) (layer F.Cu) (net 9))
 (segment (start 35.56 35.56) (end 38.0603 35.56) (width 1) (layer F.Cu) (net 9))
 (segment (start 41.18 36.83) (end 39.1797 36.83) (width 1) (layer F.Cu) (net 9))
 (segment (start 40.1797 68.6589) (end 37.5608 66.04) (width 1) (layer B.Cu) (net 6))
 (segment (start 40.1797 73.66) (end 40.1797 68.6589) (width 1) (layer B.Cu) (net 6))
 (segment (start 43.18 73.66) (end 40.1797 73.66) (width 1) (layer B.Cu) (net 6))
 (segment (start 35.56 66.04) (end 37.5608 66.04) (width 1) (layer B.Cu) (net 6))
 (segment (start 39.8103 73.66) (end 37.8103 71.66) (width 1) (layer F.Cu) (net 6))
 (segment (start 43.18 73.66) (end 39.8103 73.66) (width 1) (layer F.Cu) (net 6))
 (segment (start 35.56 71.66) (end 37.8103 71.66) (width 1) (layer F.Cu) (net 6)))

